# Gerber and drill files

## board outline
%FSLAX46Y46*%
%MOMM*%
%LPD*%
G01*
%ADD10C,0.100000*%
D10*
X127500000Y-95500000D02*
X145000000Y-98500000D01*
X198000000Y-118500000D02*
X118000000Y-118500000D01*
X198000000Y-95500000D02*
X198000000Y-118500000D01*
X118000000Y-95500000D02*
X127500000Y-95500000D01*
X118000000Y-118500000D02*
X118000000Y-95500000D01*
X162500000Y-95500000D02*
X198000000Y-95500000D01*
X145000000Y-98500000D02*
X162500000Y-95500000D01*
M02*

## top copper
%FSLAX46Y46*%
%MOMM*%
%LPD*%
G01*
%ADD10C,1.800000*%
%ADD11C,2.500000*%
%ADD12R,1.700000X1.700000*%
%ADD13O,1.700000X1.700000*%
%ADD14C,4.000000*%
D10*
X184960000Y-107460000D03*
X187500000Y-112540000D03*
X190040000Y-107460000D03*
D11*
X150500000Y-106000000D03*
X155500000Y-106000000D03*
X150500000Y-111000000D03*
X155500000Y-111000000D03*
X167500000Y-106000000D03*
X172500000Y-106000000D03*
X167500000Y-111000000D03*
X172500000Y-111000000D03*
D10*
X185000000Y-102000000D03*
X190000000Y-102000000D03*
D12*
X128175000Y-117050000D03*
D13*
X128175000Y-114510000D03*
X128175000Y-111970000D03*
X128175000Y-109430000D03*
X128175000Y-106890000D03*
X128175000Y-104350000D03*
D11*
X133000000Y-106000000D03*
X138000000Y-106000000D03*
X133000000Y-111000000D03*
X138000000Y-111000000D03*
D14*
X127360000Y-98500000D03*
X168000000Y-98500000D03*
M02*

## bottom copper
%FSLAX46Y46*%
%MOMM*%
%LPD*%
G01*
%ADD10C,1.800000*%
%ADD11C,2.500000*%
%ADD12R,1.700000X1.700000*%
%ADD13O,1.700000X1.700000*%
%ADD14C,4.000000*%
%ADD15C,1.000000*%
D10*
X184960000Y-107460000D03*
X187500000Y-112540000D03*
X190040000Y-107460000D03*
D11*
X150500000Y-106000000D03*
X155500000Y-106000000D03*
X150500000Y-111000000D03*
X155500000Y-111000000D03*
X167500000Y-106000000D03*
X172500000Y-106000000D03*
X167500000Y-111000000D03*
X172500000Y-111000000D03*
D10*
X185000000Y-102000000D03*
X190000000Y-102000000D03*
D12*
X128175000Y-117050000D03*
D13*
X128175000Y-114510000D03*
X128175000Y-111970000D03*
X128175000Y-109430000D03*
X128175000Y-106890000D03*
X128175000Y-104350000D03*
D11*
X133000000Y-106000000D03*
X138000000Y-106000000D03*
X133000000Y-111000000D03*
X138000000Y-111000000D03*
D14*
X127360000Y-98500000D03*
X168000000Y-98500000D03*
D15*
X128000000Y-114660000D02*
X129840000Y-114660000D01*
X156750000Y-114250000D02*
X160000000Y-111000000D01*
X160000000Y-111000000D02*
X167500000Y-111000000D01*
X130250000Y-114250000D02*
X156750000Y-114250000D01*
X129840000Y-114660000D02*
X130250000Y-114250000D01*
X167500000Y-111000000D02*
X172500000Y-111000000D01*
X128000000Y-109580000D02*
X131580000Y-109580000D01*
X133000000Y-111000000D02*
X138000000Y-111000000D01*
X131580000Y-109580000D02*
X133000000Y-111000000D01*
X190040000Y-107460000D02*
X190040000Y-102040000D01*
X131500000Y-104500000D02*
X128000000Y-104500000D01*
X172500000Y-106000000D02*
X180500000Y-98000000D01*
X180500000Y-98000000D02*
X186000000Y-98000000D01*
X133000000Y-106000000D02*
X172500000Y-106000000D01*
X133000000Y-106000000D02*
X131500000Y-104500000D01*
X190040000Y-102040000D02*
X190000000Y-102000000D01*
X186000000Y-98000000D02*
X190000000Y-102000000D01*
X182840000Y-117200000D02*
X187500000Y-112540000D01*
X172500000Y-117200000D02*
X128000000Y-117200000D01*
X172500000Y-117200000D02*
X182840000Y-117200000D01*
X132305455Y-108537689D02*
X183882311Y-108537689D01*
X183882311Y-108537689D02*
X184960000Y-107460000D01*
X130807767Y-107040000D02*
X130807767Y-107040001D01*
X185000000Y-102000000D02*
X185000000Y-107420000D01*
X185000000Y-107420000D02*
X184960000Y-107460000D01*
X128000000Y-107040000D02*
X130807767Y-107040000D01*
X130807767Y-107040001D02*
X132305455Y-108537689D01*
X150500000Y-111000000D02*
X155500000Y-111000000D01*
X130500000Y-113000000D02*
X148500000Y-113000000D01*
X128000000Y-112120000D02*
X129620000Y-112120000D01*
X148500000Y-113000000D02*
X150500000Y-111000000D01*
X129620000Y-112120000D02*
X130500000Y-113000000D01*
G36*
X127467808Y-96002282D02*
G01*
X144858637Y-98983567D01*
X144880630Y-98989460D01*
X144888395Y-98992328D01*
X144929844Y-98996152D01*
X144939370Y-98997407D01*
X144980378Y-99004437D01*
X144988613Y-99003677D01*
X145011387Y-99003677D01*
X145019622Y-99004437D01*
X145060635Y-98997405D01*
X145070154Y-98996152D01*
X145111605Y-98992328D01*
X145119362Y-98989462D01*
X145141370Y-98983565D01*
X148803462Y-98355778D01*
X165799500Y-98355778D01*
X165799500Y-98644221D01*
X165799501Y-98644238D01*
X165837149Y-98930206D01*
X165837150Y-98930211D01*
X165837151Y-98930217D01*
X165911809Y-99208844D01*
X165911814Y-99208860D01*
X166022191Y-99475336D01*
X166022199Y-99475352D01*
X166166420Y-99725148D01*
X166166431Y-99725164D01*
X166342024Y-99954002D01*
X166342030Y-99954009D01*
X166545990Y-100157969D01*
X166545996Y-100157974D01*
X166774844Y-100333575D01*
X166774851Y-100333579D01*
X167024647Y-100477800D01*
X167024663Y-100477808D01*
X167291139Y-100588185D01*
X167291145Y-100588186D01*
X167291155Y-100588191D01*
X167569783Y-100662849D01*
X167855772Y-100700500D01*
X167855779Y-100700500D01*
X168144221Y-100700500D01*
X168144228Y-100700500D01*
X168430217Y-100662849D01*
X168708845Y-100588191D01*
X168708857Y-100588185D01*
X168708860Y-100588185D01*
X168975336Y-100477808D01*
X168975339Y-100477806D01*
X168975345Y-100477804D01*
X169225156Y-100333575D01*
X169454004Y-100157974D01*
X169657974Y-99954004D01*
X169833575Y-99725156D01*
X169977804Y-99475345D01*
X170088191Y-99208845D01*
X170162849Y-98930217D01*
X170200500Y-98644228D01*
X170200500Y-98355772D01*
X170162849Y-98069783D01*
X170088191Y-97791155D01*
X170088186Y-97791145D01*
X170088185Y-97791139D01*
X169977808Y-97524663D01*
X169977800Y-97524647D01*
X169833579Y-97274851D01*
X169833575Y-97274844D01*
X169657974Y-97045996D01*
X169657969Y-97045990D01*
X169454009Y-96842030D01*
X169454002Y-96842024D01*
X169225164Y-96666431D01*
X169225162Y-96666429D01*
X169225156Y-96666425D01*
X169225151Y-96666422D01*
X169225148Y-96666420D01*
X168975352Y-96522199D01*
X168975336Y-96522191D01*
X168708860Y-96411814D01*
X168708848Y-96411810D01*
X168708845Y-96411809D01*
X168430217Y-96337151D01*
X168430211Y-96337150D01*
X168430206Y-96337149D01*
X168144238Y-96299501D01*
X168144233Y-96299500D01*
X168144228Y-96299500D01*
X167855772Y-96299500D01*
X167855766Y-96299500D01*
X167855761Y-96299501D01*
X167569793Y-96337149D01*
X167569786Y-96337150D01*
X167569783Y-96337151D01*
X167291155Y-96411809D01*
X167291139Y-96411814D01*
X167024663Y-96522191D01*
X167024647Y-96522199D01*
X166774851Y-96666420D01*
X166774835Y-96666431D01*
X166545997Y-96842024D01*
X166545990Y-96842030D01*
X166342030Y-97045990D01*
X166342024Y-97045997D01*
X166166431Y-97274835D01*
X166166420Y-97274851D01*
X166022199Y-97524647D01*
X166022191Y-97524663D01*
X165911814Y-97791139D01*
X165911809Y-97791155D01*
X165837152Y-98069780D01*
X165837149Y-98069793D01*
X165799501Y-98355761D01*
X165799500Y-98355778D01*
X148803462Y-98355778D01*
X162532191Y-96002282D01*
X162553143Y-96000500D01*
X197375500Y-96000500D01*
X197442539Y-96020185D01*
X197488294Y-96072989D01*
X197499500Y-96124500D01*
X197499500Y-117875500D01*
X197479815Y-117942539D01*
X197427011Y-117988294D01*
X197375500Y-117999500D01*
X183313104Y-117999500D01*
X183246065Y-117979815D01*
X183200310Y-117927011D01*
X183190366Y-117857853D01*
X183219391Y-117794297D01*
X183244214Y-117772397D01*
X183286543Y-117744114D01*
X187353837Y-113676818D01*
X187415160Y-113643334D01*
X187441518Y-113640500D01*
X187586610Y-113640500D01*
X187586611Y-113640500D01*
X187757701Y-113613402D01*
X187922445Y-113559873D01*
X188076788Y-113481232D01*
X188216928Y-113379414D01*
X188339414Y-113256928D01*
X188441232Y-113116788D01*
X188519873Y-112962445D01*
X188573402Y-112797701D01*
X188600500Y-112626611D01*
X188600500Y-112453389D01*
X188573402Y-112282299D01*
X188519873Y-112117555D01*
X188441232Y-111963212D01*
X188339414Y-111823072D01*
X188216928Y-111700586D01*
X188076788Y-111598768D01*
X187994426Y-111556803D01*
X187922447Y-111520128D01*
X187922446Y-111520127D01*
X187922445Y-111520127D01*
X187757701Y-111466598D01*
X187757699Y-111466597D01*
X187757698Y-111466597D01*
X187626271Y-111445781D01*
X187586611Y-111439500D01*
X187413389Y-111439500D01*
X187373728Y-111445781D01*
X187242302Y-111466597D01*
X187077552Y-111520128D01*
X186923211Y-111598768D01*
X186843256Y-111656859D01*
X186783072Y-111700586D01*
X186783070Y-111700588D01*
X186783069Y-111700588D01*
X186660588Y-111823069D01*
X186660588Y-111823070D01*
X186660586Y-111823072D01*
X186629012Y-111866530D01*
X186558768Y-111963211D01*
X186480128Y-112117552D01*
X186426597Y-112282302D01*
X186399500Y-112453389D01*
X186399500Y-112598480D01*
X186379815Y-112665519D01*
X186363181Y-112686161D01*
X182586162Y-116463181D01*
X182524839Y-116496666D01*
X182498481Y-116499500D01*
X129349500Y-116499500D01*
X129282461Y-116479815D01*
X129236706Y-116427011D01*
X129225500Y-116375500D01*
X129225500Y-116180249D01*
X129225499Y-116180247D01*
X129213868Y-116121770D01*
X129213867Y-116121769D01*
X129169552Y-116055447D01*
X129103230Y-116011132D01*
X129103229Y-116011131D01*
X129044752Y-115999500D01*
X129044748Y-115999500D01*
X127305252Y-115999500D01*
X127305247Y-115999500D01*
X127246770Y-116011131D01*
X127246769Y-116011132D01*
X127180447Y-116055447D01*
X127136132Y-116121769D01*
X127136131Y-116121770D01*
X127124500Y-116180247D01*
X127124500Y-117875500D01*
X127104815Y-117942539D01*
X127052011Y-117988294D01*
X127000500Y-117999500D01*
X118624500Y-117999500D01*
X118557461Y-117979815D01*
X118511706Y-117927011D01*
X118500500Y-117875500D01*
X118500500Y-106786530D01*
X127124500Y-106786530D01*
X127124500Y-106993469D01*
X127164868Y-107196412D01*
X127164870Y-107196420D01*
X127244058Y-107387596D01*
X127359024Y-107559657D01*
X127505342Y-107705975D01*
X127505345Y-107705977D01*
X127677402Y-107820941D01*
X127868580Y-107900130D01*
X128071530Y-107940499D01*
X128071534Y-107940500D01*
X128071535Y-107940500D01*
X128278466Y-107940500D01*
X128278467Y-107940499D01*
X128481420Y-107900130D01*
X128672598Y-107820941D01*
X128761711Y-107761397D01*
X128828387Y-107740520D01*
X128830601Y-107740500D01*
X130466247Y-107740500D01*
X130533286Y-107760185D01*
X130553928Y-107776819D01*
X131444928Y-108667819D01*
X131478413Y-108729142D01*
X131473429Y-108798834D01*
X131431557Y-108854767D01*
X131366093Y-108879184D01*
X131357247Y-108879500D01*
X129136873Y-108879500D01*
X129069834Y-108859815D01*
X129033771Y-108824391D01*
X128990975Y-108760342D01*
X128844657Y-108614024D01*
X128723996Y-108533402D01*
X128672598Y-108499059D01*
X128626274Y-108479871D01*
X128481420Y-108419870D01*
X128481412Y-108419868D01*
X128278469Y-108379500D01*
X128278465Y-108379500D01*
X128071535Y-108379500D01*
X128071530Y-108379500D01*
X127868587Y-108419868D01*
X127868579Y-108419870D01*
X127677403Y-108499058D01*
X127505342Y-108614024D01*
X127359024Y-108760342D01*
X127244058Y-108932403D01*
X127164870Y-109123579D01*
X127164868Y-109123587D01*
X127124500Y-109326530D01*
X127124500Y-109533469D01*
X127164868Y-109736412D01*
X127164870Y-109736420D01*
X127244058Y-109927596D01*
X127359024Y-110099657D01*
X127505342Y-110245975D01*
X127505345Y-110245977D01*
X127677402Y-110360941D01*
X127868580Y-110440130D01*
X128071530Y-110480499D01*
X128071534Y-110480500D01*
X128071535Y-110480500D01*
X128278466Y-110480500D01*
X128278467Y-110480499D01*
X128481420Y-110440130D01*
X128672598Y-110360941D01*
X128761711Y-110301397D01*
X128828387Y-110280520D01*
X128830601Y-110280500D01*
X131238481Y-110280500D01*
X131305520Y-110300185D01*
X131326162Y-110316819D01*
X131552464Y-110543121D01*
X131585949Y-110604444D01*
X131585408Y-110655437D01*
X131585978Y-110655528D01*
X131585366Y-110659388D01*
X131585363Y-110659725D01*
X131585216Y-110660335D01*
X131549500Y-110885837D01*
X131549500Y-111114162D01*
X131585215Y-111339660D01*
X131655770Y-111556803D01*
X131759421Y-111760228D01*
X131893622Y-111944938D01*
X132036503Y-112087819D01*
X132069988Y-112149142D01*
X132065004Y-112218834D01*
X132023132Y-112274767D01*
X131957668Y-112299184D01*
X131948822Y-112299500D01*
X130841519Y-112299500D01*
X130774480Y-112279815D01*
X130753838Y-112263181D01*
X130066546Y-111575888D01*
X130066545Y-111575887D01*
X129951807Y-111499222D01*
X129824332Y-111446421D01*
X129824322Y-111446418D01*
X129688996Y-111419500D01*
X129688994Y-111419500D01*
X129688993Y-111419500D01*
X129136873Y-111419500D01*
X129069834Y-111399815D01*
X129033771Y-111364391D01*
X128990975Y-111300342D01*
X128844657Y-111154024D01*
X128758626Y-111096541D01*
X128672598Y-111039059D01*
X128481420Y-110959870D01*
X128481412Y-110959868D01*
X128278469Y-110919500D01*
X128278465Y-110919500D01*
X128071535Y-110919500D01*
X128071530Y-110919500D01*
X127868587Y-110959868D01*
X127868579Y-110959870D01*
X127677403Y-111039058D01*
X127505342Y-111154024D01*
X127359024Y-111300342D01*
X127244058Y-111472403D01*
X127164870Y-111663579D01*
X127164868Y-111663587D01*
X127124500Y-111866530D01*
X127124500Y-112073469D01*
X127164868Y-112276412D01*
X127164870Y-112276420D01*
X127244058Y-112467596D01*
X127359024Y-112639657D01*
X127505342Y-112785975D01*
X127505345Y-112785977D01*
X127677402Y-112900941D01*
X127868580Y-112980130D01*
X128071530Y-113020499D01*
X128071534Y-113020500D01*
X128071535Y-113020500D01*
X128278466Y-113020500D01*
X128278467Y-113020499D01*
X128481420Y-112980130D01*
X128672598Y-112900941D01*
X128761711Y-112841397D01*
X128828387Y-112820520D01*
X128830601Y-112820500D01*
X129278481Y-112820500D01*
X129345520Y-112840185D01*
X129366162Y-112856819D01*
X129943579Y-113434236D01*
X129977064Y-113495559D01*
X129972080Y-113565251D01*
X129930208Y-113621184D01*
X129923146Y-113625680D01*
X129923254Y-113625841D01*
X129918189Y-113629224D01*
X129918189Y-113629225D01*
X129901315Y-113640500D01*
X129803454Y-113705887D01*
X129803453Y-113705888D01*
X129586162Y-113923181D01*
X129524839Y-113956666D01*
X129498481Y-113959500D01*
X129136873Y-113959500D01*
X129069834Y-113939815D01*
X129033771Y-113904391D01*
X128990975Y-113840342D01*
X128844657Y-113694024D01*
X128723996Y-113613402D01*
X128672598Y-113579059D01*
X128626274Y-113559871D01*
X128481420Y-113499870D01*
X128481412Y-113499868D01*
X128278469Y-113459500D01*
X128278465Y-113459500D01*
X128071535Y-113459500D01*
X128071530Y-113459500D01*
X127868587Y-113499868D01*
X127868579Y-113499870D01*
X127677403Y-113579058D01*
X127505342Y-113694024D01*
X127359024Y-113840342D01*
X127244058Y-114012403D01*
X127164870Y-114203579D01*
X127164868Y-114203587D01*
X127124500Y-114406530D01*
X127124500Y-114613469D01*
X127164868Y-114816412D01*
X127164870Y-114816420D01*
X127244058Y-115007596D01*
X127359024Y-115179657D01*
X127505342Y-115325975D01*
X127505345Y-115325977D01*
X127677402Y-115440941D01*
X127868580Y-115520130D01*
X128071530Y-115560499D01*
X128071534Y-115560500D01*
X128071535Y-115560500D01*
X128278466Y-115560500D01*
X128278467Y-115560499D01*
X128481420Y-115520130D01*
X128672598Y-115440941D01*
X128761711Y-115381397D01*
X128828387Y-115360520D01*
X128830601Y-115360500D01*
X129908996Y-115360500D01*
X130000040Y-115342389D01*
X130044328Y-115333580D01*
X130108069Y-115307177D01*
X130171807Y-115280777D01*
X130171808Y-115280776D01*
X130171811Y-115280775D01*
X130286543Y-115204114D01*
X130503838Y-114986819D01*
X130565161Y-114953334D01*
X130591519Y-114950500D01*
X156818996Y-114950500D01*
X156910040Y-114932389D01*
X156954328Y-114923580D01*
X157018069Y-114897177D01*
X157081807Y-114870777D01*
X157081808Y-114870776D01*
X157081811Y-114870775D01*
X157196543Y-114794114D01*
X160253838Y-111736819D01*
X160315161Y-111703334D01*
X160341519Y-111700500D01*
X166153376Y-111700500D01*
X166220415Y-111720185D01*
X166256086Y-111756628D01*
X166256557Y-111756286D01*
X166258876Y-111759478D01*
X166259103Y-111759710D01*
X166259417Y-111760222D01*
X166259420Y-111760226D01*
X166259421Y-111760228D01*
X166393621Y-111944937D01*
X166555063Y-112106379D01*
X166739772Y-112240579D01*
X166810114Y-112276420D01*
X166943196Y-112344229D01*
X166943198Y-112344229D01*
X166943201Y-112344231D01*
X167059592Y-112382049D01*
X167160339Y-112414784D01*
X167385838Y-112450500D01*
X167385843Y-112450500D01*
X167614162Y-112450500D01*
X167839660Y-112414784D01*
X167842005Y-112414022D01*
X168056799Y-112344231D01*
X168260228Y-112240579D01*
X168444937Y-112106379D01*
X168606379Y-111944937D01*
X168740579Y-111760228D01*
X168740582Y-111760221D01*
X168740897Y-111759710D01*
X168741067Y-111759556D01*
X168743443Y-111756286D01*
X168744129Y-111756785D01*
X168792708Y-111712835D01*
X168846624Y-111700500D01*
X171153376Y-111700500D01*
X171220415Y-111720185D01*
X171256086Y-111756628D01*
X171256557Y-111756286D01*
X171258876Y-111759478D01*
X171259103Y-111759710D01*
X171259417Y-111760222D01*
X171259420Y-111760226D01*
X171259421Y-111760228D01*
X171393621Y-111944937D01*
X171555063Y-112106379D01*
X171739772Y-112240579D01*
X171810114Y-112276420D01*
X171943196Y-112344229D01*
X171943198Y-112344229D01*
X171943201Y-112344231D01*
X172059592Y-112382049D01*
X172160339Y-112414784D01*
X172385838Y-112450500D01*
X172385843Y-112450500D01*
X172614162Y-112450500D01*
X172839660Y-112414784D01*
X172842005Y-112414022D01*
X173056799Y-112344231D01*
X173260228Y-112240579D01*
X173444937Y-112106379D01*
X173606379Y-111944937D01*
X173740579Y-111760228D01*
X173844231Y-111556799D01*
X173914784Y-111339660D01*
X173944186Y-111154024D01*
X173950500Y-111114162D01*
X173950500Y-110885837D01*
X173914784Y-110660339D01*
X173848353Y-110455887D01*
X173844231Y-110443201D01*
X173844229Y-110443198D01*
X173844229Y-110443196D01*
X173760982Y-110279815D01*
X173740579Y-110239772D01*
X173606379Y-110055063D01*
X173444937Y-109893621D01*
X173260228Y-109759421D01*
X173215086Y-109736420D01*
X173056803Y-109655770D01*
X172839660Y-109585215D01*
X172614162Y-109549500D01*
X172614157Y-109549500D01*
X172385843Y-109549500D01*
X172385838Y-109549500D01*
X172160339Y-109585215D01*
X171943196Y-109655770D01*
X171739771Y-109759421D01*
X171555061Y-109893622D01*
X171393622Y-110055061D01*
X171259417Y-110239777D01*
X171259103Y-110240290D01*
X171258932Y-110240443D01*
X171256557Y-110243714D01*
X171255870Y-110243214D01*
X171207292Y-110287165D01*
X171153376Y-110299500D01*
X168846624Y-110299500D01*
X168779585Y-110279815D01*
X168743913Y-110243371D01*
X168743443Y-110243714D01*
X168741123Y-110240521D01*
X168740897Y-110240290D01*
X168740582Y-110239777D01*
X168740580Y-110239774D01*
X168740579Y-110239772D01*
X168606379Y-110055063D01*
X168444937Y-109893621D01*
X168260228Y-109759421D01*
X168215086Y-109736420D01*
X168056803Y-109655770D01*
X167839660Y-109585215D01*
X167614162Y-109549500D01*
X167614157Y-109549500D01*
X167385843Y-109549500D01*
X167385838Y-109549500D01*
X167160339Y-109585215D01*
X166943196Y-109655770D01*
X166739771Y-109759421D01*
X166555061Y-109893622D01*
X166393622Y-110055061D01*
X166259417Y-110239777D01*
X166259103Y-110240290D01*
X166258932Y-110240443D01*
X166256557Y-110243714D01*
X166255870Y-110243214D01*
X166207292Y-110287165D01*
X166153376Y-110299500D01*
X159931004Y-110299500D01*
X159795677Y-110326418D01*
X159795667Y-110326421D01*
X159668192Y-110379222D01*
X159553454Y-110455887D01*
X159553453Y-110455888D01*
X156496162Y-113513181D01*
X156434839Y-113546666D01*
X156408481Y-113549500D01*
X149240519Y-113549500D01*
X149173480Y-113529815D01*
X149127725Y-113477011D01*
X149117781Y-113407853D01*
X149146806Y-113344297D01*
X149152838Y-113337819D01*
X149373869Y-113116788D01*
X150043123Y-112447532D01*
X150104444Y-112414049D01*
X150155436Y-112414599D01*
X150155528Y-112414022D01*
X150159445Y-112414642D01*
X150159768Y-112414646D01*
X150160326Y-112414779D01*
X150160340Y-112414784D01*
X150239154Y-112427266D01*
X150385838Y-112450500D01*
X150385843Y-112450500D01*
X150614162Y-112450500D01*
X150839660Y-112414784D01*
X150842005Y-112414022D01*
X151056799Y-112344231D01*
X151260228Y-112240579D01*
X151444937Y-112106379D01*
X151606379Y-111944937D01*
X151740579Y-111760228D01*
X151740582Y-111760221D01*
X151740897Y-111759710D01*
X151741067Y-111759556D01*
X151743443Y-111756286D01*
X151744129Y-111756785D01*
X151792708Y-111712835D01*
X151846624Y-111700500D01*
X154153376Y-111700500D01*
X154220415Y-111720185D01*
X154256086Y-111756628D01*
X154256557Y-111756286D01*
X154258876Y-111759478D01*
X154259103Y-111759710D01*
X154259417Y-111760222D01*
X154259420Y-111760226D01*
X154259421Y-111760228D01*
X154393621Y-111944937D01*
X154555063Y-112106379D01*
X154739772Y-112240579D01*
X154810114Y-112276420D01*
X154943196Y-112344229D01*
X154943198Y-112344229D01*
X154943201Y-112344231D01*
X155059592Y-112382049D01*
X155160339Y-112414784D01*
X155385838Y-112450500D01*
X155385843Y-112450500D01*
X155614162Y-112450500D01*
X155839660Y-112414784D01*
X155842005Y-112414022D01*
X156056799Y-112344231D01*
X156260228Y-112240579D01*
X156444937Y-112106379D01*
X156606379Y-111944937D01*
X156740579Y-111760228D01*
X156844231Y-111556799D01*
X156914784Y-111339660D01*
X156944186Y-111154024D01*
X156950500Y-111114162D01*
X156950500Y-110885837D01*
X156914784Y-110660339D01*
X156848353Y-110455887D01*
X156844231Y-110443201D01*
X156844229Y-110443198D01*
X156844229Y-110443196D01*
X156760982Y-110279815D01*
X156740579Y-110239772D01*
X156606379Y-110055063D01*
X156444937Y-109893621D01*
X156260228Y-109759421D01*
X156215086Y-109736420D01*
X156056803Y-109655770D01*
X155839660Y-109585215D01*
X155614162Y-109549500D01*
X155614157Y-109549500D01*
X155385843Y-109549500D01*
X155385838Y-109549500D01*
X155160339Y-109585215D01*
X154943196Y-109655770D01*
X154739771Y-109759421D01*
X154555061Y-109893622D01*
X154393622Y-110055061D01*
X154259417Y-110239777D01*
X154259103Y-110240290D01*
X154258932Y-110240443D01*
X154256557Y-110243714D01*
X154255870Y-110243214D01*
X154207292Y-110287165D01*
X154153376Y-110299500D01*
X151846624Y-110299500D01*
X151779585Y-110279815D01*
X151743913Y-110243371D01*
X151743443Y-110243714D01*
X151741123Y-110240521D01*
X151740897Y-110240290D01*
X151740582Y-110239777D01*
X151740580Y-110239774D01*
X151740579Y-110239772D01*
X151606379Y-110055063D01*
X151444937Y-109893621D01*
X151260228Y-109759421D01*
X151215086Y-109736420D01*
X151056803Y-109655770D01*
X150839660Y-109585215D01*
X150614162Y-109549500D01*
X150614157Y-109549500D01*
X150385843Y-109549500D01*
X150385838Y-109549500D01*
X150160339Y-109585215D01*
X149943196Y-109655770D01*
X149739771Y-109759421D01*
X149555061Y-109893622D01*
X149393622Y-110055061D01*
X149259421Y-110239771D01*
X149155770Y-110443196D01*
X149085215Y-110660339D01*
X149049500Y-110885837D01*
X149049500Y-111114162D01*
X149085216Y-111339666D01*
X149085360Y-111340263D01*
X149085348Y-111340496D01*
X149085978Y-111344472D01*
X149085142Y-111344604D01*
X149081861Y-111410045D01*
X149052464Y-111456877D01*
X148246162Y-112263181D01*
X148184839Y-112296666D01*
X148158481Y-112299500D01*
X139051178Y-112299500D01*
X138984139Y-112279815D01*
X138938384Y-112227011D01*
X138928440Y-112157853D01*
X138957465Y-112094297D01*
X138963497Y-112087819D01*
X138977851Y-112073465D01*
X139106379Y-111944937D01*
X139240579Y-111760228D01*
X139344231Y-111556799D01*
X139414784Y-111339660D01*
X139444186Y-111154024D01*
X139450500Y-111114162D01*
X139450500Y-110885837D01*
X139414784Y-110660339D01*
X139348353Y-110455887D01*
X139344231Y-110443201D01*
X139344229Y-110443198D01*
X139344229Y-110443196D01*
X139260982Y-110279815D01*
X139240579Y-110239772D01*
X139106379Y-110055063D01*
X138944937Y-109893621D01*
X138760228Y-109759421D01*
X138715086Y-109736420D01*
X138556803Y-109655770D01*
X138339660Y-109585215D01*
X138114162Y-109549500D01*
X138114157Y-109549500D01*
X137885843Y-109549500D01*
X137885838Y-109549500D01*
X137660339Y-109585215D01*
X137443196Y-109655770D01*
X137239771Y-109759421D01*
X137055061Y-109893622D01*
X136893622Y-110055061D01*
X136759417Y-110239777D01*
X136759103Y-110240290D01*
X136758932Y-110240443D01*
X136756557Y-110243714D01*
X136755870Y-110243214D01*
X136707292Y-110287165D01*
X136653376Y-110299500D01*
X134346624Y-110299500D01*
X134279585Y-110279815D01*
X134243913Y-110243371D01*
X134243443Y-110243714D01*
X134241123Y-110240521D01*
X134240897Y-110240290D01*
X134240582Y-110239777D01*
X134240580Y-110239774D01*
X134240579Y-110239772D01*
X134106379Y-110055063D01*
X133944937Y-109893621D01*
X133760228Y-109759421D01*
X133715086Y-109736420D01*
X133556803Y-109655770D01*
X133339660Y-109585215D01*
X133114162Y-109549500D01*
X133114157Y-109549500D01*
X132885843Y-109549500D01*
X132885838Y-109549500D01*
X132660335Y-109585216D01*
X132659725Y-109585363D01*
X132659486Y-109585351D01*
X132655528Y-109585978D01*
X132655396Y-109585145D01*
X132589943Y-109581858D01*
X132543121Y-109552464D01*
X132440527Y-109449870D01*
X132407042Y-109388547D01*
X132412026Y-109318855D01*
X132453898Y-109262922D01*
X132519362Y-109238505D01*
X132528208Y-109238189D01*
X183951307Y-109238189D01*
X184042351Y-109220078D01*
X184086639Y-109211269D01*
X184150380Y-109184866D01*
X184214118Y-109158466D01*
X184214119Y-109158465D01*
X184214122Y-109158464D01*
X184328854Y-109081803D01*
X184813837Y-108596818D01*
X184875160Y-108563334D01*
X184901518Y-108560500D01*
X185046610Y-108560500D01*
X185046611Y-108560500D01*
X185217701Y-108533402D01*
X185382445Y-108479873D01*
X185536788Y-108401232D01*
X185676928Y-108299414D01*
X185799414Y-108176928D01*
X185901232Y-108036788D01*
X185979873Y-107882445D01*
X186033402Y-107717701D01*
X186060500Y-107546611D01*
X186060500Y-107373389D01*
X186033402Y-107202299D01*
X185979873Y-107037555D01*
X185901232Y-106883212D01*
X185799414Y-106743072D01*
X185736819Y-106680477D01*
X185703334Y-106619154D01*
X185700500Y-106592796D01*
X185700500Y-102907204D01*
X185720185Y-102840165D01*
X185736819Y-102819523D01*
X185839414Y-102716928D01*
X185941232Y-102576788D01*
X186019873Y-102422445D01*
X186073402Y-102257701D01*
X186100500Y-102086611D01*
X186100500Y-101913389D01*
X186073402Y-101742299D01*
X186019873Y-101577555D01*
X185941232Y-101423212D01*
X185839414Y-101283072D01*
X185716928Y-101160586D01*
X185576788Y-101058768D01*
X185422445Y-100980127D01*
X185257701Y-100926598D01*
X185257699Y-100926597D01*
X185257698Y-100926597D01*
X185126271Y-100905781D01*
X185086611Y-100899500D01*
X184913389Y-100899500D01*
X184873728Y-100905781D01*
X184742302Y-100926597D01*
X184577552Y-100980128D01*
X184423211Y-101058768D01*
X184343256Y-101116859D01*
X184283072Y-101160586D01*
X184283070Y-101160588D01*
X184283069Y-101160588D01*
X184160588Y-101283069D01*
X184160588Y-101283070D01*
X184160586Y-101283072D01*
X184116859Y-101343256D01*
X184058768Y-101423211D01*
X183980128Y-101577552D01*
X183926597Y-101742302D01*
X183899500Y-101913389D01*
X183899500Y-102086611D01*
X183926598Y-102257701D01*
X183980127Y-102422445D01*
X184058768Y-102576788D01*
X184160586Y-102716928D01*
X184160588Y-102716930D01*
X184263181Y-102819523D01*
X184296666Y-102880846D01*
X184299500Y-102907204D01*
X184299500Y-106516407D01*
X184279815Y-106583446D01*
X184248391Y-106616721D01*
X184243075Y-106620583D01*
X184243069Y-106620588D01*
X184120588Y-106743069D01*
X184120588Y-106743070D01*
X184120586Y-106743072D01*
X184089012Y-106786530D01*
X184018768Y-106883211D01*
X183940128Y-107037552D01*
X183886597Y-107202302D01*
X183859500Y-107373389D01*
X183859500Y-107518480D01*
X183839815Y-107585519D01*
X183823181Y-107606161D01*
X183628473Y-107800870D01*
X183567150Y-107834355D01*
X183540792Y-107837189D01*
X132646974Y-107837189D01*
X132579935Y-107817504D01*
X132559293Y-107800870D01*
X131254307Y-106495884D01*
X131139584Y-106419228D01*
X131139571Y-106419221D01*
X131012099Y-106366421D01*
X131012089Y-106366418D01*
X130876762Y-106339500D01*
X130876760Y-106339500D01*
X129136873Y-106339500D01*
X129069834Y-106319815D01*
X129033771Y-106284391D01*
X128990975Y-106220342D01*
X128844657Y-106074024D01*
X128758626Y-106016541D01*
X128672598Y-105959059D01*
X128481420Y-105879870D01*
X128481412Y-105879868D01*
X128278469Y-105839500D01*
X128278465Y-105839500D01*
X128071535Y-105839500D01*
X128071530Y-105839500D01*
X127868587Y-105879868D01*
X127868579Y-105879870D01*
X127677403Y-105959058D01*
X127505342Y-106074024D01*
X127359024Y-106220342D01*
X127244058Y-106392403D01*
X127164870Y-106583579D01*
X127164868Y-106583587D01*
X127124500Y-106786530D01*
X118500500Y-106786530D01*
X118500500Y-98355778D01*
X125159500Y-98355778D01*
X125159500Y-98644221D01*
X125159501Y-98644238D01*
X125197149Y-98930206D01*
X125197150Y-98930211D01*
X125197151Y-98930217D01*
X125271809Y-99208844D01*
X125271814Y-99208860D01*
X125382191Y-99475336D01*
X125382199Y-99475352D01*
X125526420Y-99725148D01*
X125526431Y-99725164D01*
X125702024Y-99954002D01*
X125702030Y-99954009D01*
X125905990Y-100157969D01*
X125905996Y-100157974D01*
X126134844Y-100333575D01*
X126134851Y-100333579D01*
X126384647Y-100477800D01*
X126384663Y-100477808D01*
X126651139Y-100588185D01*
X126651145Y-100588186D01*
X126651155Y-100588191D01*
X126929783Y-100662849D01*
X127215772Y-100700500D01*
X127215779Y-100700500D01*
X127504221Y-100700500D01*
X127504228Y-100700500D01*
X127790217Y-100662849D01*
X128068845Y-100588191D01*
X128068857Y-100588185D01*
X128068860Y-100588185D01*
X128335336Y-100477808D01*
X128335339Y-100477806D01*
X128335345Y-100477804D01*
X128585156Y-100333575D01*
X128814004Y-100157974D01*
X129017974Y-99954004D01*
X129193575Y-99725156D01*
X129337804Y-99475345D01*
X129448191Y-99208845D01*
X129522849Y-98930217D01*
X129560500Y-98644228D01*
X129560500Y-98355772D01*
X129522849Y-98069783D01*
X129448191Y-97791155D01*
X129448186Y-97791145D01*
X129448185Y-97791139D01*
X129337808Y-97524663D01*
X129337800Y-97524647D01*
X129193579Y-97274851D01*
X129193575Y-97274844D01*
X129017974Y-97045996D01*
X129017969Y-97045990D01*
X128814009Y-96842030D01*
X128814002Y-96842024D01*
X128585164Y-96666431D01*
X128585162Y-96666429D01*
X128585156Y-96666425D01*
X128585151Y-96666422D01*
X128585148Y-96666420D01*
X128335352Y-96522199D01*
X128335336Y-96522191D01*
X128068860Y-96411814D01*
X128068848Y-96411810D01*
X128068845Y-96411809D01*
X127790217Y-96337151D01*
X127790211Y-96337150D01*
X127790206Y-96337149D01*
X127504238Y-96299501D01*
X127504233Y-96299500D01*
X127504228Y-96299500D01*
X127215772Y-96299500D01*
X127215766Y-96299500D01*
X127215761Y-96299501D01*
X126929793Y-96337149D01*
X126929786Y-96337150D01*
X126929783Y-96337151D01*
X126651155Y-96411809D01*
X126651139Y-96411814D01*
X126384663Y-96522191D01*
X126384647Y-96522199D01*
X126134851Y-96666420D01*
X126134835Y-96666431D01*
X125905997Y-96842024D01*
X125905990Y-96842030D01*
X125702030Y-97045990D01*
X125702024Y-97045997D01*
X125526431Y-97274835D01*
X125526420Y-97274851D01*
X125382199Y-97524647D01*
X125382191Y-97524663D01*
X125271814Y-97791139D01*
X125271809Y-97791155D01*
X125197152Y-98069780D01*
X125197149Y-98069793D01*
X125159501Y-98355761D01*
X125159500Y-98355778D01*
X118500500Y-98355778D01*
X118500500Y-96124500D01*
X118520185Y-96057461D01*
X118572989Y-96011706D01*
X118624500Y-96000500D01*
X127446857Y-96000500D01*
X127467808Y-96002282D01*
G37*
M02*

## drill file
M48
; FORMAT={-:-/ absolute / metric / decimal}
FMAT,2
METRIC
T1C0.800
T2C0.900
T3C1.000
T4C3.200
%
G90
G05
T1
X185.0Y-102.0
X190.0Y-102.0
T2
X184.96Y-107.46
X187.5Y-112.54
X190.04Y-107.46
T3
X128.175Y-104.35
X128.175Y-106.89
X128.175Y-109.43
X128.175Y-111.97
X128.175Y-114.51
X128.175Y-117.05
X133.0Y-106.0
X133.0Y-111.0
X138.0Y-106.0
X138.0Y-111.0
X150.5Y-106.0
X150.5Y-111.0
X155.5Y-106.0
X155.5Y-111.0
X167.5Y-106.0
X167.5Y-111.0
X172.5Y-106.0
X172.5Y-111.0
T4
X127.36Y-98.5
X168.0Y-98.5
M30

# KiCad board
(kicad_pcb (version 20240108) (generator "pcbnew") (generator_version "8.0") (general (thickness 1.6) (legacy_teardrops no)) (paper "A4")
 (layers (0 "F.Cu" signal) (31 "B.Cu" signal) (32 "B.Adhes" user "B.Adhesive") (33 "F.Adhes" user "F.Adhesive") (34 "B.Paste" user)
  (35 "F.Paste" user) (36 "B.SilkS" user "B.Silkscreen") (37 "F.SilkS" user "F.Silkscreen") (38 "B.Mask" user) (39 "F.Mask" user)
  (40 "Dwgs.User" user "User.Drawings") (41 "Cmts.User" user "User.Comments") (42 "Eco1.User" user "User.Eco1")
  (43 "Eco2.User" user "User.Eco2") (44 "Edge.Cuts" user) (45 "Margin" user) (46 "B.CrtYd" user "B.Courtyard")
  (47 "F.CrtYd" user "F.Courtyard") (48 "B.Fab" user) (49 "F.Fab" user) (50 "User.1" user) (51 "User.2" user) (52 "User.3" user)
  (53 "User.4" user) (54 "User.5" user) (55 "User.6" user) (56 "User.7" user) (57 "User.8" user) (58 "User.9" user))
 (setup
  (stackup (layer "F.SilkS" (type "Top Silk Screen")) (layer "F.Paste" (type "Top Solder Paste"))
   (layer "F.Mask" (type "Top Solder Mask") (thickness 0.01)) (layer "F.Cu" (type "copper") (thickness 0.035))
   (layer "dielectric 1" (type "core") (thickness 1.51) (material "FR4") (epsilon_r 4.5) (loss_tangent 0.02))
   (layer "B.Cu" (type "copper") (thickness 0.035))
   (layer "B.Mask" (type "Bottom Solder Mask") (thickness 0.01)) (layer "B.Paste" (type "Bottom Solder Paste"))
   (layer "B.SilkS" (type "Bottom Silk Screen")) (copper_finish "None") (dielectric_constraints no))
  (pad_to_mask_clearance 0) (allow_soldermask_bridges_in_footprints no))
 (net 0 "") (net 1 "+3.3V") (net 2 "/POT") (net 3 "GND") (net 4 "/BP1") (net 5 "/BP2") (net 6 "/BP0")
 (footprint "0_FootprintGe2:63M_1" (layer "F.Cu") (at 187.5 110 180)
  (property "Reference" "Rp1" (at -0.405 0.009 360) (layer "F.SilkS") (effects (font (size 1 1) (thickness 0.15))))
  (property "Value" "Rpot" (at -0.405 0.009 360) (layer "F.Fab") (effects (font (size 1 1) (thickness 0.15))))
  (pad "1" thru_hole circle (at 2.54 2.54 180) (size 1.8 1.8) (drill 0.9) (layers "*.Cu" "*.Mask") (remove_unused_layers no) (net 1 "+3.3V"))
  (pad "2" thru_hole circle (at 0 -2.54 180) (size 1.8 1.8) (drill 0.9) (layers "*.Cu" "*.Mask") (remove_unused_layers no) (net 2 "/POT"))
  (pad "3" thru_hole circle (at -2.54 2.54 180) (size 1.8 1.8) (drill 0.9) (layers "*.Cu" "*.Mask") (remove_unused_layers no) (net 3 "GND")))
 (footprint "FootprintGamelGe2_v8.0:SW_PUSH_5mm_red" (layer "F.Cu") (at 150.5 106)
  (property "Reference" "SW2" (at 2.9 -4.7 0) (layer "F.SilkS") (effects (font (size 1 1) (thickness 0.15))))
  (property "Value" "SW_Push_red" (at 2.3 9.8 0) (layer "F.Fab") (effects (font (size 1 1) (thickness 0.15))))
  (pad "1" thru_hole circle (at 0 0 90) (size 2.5 2.5) (drill 1) (layers "*.Cu" "*.Mask") (remove_unused_layers no) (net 3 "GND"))
  (pad "1" thru_hole circle (at 5 0 90) (size 2.5 2.5) (drill 1) (layers "*.Cu" "*.Mask") (remove_unused_layers no) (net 3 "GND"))
  (pad "2" thru_hole circle (at 0 5 90) (size 2.5 2.5) (drill 1) (layers "*.Cu" "*.Mask") (remove_unused_layers no) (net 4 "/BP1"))
  (pad "2" thru_hole circle (at 5 5 90) (size 2.5 2.5) (drill 1) (layers "*.Cu" "*.Mask") (remove_unused_layers no) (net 4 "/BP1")))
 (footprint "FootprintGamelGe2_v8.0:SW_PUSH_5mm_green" (layer "F.Cu") (at 167.5 106)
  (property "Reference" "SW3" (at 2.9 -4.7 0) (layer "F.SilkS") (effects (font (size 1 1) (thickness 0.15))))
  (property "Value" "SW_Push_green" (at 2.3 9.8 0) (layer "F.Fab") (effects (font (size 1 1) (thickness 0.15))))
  (pad "1" thru_hole circle (at 0 0 90) (size 2.5 2.5) (drill 1) (layers "*.Cu" "*.Mask") (remove_unused_layers no) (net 3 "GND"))
  (pad "1" thru_hole circle (at 5 0 90) (size 2.5 2.5) (drill 1) (layers "*.Cu" "*.Mask") (remove_unused_layers no) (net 3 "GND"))
  (pad "2" thru_hole circle (at 0 5 90) (size 2.5 2.5) (drill 1) (layers "*.Cu" "*.Mask") (remove_unused_layers no) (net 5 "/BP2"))
  (pad "2" thru_hole circle (at 5 5 90) (size 2.5 2.5) (drill 1) (layers "*.Cu" "*.Mask") (remove_unused_layers no) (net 5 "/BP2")))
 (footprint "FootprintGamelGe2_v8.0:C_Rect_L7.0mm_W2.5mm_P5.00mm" (layer "F.Cu") (at 185 102)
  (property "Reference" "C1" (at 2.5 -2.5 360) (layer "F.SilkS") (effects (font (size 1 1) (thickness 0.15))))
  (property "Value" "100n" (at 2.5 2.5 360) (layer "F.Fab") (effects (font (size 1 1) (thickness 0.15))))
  (pad "1" thru_hole circle (at 0 0) (size 1.8 1.8) (drill 0.8) (layers "*.Cu" "*.Mask") (remove_unused_layers no) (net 1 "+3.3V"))
  (pad "2" thru_hole circle (at 5 0) (size 1.8 1.8) (drill 0.8) (layers "*.Cu" "*.Mask") (remove_unused_layers no) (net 3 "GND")))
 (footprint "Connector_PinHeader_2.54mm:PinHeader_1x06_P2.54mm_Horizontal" (layer "F.Cu") (at 128.175 117.05 180)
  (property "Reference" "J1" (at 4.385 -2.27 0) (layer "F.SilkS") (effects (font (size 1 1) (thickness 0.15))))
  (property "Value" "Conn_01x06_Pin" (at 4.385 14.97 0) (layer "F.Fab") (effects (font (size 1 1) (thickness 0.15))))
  (pad "1" thru_hole rect (at 0 0 180) (size 1.7 1.7) (drill 1) (layers "*.Cu" "*.Mask") (remove_unused_layers no) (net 2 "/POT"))
  (pad "2" thru_hole oval (at 0 2.54 180) (size 1.7 1.7) (drill 1) (layers "*.Cu" "*.Mask") (remove_unused_layers no) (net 5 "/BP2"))
  (pad "3" thru_hole oval (at 0 5.08 180) (size 1.7 1.7) (drill 1) (layers "*.Cu" "*.Mask") (remove_unused_layers no) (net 4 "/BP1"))
  (pad "4" thru_hole oval (at 0 7.62 180) (size 1.7 1.7) (drill 1) (layers "*.Cu" "*.Mask") (remove_unused_layers no) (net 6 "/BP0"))
  (pad "5" thru_hole oval (at 0 10.16 180) (size 1.7 1.7) (drill 1) (layers "*.Cu" "*.Mask") (remove_unused_layers no) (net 1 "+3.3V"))
  (pad "6" thru_hole oval (at 0 12.7 180) (size 1.7 1.7) (drill 1) (layers "*.Cu" "*.Mask") (remove_unused_layers no) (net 3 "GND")))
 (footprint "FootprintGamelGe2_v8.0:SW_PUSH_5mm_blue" (layer "F.Cu") (at 133 106)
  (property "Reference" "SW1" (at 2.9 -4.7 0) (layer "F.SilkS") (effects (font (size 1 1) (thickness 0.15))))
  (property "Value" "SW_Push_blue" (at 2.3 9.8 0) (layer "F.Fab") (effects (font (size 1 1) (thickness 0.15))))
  (pad "1" thru_hole circle (at 0 0 90) (size 2.5 2.5) (drill 1) (layers "*.Cu" "*.Mask") (remove_unused_layers no) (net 3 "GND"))
  (pad "1" thru_hole circle (at 5 0 90) (size 2.5 2.5) (drill 1) (layers "*.Cu" "*.Mask") (remove_unused_layers no) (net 3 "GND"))
  (pad "2" thru_hole circle (at 0 5 90) (size 2.5 2.5) (drill 1) (layers "*.Cu" "*.Mask") (remove_unused_layers no) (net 6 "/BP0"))
  (pad "2" thru_hole circle (at 5 5 90) (size 2.5 2.5) (drill 1) (layers "*.Cu" "*.Mask") (remove_unused_layers no) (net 6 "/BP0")))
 (gr_line (start 127.5 95.5) (end 145 98.5) (stroke (width 0.1) (type default)) (layer "Edge.Cuts"))
 (gr_line (start 198 118.5) (end 118 118.5) (stroke (width 0.1) (type default)) (layer "Edge.Cuts"))
 (gr_line (start 198 95.5) (end 198 118.5) (stroke (width 0.1) (type default)) (layer "Edge.Cuts"))
 (gr_line (start 118 95.5) (end 127.5 95.5) (stroke (width 0.1) (type default)) (layer "Edge.Cuts"))
 (gr_line (start 118 118.5) (end 118 95.5) (stroke (width 0.1) (type default)) (layer "Edge.Cuts"))
 (gr_line (start 162.5 95.5) (end 198 95.5) (stroke (width 0.1) (type default)) (layer "Edge.Cuts"))
 (gr_line (start 145 98.5) (end 162.5 95.5) (stroke (width 0.1) (type default)) (layer "Edge.Cuts"))
 (via (at 127.36 98.5) (size 4) (drill 3.2) (layers "F.Cu" "B.Cu") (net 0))
 (via (at 168 98.5) (size 4) (drill 3.2) (layers "F.Cu" "B.Cu") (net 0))
 (segment (start 128 114.66) (end 129.84 114.66) (width 1) (layer "B.Cu") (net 5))
 (segment (start 156.75 114.25) (end 160 111) (width 1) (layer "B.Cu") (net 5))
 (segment (start 160 111) (end 167.5 111) (width 1) (layer "B.Cu") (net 5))
 (segment (start 130.25 114.25) (end 156.75 114.25) (width 1) (layer "B.Cu") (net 5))
 (segment (start 129.84 114.66) (end 130.25 114.25) (width 1) (layer "B.Cu") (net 5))
 (segment (start 167.5 111) (end 172.5 111) (width 1) (layer "B.Cu") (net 5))
 (segment (start 128 109.58) (end 131.58 109.58) (width 1) (layer "B.Cu") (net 6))
 (segment (start 133 111) (end 138 111) (width 1) (layer "B.Cu") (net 6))
 (segment (start 131.58 109.58) (end 133 111) (width 1) (layer "B.Cu") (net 6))
 (segment (start 190.04 107.46) (end 190.04 102.04) (width 1) (layer "B.Cu") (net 3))
 (segment (start 131.5 104.5) (end 128 104.5) (width 1) (layer "B.Cu") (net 3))
 (segment (start 172.5 106) (end 180.5 98) (width 1) (layer "B.Cu") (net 3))
 (segment (start 180.5 98) (end 186 98) (width 1) (layer "B.Cu") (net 3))
 (segment (start 133 106) (end 172.5 106) (width 1) (layer "B.Cu") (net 3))
 (segment (start 133 106) (end 131.5 104.5) (width 1) (layer "B.Cu") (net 3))
 (segment (start 190.04 102.04) (end 190 102) (width 1) (layer "B.Cu") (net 3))
 (segment (start 186 98) (end 190 102) (width 1) (layer "B.Cu") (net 3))
 (segment (start 182.84 117.2) (end 187.5 112.54) (width 1) (layer "B.Cu") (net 2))
 (segment (start 172.5 117.2) (end 128 117.2) (width 1) (layer "B.Cu") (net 2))
 (segment (start 172.5 117.2) (end 182.84 117.2) (width 1) (layer "B.Cu") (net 2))
 (segment (start 132.305455 108.537689) (end 183.882311 108.537689) (width 1) (layer "B.Cu") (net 1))
 (segment (start 183.882311 108.537689) (end 184.96 107.46) (width 1) (layer "B.Cu") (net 1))
 (segment (start 130.807767 107.04) (end 130.807767 107.040001) (width 1) (layer "B.Cu") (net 1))
 (segment (start 185 102) (end 185 107.42) (width 1) (layer "B.Cu") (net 1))
 (segment (start 185 107.42) (end 184.96 107.46) (width 1) (layer "B.Cu") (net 1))
 (segment (start 128 107.04) (end 130.807767 107.04) (width 1) (layer "B.Cu") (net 1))
 (segment (start 130.807767 107.040001) (end 132.305455 108.537689) (width 1) (layer "B.Cu") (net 1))
 (segment (start 150.5 111) (end 155.5 111) (width 1) (layer "B.Cu") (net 4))
 (segment (start 130.5 113) (end 148.5 113) (width 1) (layer "B.Cu") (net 4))
 (segment (start 128 112.12) (end 129.62 112.12) (width 1) (layer "B.Cu") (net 4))
 (segment (start 148.5 113) (end 150.5 111) (width 1) (layer "B.Cu") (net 4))
 (segment (start 129.62 112.12) (end 130.5 113) (width 1) (layer "B.Cu") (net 4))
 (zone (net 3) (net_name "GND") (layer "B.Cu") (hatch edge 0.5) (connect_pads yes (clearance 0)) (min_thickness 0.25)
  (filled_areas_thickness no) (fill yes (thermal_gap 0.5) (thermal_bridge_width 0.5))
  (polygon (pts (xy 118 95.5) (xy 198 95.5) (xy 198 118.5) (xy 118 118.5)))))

